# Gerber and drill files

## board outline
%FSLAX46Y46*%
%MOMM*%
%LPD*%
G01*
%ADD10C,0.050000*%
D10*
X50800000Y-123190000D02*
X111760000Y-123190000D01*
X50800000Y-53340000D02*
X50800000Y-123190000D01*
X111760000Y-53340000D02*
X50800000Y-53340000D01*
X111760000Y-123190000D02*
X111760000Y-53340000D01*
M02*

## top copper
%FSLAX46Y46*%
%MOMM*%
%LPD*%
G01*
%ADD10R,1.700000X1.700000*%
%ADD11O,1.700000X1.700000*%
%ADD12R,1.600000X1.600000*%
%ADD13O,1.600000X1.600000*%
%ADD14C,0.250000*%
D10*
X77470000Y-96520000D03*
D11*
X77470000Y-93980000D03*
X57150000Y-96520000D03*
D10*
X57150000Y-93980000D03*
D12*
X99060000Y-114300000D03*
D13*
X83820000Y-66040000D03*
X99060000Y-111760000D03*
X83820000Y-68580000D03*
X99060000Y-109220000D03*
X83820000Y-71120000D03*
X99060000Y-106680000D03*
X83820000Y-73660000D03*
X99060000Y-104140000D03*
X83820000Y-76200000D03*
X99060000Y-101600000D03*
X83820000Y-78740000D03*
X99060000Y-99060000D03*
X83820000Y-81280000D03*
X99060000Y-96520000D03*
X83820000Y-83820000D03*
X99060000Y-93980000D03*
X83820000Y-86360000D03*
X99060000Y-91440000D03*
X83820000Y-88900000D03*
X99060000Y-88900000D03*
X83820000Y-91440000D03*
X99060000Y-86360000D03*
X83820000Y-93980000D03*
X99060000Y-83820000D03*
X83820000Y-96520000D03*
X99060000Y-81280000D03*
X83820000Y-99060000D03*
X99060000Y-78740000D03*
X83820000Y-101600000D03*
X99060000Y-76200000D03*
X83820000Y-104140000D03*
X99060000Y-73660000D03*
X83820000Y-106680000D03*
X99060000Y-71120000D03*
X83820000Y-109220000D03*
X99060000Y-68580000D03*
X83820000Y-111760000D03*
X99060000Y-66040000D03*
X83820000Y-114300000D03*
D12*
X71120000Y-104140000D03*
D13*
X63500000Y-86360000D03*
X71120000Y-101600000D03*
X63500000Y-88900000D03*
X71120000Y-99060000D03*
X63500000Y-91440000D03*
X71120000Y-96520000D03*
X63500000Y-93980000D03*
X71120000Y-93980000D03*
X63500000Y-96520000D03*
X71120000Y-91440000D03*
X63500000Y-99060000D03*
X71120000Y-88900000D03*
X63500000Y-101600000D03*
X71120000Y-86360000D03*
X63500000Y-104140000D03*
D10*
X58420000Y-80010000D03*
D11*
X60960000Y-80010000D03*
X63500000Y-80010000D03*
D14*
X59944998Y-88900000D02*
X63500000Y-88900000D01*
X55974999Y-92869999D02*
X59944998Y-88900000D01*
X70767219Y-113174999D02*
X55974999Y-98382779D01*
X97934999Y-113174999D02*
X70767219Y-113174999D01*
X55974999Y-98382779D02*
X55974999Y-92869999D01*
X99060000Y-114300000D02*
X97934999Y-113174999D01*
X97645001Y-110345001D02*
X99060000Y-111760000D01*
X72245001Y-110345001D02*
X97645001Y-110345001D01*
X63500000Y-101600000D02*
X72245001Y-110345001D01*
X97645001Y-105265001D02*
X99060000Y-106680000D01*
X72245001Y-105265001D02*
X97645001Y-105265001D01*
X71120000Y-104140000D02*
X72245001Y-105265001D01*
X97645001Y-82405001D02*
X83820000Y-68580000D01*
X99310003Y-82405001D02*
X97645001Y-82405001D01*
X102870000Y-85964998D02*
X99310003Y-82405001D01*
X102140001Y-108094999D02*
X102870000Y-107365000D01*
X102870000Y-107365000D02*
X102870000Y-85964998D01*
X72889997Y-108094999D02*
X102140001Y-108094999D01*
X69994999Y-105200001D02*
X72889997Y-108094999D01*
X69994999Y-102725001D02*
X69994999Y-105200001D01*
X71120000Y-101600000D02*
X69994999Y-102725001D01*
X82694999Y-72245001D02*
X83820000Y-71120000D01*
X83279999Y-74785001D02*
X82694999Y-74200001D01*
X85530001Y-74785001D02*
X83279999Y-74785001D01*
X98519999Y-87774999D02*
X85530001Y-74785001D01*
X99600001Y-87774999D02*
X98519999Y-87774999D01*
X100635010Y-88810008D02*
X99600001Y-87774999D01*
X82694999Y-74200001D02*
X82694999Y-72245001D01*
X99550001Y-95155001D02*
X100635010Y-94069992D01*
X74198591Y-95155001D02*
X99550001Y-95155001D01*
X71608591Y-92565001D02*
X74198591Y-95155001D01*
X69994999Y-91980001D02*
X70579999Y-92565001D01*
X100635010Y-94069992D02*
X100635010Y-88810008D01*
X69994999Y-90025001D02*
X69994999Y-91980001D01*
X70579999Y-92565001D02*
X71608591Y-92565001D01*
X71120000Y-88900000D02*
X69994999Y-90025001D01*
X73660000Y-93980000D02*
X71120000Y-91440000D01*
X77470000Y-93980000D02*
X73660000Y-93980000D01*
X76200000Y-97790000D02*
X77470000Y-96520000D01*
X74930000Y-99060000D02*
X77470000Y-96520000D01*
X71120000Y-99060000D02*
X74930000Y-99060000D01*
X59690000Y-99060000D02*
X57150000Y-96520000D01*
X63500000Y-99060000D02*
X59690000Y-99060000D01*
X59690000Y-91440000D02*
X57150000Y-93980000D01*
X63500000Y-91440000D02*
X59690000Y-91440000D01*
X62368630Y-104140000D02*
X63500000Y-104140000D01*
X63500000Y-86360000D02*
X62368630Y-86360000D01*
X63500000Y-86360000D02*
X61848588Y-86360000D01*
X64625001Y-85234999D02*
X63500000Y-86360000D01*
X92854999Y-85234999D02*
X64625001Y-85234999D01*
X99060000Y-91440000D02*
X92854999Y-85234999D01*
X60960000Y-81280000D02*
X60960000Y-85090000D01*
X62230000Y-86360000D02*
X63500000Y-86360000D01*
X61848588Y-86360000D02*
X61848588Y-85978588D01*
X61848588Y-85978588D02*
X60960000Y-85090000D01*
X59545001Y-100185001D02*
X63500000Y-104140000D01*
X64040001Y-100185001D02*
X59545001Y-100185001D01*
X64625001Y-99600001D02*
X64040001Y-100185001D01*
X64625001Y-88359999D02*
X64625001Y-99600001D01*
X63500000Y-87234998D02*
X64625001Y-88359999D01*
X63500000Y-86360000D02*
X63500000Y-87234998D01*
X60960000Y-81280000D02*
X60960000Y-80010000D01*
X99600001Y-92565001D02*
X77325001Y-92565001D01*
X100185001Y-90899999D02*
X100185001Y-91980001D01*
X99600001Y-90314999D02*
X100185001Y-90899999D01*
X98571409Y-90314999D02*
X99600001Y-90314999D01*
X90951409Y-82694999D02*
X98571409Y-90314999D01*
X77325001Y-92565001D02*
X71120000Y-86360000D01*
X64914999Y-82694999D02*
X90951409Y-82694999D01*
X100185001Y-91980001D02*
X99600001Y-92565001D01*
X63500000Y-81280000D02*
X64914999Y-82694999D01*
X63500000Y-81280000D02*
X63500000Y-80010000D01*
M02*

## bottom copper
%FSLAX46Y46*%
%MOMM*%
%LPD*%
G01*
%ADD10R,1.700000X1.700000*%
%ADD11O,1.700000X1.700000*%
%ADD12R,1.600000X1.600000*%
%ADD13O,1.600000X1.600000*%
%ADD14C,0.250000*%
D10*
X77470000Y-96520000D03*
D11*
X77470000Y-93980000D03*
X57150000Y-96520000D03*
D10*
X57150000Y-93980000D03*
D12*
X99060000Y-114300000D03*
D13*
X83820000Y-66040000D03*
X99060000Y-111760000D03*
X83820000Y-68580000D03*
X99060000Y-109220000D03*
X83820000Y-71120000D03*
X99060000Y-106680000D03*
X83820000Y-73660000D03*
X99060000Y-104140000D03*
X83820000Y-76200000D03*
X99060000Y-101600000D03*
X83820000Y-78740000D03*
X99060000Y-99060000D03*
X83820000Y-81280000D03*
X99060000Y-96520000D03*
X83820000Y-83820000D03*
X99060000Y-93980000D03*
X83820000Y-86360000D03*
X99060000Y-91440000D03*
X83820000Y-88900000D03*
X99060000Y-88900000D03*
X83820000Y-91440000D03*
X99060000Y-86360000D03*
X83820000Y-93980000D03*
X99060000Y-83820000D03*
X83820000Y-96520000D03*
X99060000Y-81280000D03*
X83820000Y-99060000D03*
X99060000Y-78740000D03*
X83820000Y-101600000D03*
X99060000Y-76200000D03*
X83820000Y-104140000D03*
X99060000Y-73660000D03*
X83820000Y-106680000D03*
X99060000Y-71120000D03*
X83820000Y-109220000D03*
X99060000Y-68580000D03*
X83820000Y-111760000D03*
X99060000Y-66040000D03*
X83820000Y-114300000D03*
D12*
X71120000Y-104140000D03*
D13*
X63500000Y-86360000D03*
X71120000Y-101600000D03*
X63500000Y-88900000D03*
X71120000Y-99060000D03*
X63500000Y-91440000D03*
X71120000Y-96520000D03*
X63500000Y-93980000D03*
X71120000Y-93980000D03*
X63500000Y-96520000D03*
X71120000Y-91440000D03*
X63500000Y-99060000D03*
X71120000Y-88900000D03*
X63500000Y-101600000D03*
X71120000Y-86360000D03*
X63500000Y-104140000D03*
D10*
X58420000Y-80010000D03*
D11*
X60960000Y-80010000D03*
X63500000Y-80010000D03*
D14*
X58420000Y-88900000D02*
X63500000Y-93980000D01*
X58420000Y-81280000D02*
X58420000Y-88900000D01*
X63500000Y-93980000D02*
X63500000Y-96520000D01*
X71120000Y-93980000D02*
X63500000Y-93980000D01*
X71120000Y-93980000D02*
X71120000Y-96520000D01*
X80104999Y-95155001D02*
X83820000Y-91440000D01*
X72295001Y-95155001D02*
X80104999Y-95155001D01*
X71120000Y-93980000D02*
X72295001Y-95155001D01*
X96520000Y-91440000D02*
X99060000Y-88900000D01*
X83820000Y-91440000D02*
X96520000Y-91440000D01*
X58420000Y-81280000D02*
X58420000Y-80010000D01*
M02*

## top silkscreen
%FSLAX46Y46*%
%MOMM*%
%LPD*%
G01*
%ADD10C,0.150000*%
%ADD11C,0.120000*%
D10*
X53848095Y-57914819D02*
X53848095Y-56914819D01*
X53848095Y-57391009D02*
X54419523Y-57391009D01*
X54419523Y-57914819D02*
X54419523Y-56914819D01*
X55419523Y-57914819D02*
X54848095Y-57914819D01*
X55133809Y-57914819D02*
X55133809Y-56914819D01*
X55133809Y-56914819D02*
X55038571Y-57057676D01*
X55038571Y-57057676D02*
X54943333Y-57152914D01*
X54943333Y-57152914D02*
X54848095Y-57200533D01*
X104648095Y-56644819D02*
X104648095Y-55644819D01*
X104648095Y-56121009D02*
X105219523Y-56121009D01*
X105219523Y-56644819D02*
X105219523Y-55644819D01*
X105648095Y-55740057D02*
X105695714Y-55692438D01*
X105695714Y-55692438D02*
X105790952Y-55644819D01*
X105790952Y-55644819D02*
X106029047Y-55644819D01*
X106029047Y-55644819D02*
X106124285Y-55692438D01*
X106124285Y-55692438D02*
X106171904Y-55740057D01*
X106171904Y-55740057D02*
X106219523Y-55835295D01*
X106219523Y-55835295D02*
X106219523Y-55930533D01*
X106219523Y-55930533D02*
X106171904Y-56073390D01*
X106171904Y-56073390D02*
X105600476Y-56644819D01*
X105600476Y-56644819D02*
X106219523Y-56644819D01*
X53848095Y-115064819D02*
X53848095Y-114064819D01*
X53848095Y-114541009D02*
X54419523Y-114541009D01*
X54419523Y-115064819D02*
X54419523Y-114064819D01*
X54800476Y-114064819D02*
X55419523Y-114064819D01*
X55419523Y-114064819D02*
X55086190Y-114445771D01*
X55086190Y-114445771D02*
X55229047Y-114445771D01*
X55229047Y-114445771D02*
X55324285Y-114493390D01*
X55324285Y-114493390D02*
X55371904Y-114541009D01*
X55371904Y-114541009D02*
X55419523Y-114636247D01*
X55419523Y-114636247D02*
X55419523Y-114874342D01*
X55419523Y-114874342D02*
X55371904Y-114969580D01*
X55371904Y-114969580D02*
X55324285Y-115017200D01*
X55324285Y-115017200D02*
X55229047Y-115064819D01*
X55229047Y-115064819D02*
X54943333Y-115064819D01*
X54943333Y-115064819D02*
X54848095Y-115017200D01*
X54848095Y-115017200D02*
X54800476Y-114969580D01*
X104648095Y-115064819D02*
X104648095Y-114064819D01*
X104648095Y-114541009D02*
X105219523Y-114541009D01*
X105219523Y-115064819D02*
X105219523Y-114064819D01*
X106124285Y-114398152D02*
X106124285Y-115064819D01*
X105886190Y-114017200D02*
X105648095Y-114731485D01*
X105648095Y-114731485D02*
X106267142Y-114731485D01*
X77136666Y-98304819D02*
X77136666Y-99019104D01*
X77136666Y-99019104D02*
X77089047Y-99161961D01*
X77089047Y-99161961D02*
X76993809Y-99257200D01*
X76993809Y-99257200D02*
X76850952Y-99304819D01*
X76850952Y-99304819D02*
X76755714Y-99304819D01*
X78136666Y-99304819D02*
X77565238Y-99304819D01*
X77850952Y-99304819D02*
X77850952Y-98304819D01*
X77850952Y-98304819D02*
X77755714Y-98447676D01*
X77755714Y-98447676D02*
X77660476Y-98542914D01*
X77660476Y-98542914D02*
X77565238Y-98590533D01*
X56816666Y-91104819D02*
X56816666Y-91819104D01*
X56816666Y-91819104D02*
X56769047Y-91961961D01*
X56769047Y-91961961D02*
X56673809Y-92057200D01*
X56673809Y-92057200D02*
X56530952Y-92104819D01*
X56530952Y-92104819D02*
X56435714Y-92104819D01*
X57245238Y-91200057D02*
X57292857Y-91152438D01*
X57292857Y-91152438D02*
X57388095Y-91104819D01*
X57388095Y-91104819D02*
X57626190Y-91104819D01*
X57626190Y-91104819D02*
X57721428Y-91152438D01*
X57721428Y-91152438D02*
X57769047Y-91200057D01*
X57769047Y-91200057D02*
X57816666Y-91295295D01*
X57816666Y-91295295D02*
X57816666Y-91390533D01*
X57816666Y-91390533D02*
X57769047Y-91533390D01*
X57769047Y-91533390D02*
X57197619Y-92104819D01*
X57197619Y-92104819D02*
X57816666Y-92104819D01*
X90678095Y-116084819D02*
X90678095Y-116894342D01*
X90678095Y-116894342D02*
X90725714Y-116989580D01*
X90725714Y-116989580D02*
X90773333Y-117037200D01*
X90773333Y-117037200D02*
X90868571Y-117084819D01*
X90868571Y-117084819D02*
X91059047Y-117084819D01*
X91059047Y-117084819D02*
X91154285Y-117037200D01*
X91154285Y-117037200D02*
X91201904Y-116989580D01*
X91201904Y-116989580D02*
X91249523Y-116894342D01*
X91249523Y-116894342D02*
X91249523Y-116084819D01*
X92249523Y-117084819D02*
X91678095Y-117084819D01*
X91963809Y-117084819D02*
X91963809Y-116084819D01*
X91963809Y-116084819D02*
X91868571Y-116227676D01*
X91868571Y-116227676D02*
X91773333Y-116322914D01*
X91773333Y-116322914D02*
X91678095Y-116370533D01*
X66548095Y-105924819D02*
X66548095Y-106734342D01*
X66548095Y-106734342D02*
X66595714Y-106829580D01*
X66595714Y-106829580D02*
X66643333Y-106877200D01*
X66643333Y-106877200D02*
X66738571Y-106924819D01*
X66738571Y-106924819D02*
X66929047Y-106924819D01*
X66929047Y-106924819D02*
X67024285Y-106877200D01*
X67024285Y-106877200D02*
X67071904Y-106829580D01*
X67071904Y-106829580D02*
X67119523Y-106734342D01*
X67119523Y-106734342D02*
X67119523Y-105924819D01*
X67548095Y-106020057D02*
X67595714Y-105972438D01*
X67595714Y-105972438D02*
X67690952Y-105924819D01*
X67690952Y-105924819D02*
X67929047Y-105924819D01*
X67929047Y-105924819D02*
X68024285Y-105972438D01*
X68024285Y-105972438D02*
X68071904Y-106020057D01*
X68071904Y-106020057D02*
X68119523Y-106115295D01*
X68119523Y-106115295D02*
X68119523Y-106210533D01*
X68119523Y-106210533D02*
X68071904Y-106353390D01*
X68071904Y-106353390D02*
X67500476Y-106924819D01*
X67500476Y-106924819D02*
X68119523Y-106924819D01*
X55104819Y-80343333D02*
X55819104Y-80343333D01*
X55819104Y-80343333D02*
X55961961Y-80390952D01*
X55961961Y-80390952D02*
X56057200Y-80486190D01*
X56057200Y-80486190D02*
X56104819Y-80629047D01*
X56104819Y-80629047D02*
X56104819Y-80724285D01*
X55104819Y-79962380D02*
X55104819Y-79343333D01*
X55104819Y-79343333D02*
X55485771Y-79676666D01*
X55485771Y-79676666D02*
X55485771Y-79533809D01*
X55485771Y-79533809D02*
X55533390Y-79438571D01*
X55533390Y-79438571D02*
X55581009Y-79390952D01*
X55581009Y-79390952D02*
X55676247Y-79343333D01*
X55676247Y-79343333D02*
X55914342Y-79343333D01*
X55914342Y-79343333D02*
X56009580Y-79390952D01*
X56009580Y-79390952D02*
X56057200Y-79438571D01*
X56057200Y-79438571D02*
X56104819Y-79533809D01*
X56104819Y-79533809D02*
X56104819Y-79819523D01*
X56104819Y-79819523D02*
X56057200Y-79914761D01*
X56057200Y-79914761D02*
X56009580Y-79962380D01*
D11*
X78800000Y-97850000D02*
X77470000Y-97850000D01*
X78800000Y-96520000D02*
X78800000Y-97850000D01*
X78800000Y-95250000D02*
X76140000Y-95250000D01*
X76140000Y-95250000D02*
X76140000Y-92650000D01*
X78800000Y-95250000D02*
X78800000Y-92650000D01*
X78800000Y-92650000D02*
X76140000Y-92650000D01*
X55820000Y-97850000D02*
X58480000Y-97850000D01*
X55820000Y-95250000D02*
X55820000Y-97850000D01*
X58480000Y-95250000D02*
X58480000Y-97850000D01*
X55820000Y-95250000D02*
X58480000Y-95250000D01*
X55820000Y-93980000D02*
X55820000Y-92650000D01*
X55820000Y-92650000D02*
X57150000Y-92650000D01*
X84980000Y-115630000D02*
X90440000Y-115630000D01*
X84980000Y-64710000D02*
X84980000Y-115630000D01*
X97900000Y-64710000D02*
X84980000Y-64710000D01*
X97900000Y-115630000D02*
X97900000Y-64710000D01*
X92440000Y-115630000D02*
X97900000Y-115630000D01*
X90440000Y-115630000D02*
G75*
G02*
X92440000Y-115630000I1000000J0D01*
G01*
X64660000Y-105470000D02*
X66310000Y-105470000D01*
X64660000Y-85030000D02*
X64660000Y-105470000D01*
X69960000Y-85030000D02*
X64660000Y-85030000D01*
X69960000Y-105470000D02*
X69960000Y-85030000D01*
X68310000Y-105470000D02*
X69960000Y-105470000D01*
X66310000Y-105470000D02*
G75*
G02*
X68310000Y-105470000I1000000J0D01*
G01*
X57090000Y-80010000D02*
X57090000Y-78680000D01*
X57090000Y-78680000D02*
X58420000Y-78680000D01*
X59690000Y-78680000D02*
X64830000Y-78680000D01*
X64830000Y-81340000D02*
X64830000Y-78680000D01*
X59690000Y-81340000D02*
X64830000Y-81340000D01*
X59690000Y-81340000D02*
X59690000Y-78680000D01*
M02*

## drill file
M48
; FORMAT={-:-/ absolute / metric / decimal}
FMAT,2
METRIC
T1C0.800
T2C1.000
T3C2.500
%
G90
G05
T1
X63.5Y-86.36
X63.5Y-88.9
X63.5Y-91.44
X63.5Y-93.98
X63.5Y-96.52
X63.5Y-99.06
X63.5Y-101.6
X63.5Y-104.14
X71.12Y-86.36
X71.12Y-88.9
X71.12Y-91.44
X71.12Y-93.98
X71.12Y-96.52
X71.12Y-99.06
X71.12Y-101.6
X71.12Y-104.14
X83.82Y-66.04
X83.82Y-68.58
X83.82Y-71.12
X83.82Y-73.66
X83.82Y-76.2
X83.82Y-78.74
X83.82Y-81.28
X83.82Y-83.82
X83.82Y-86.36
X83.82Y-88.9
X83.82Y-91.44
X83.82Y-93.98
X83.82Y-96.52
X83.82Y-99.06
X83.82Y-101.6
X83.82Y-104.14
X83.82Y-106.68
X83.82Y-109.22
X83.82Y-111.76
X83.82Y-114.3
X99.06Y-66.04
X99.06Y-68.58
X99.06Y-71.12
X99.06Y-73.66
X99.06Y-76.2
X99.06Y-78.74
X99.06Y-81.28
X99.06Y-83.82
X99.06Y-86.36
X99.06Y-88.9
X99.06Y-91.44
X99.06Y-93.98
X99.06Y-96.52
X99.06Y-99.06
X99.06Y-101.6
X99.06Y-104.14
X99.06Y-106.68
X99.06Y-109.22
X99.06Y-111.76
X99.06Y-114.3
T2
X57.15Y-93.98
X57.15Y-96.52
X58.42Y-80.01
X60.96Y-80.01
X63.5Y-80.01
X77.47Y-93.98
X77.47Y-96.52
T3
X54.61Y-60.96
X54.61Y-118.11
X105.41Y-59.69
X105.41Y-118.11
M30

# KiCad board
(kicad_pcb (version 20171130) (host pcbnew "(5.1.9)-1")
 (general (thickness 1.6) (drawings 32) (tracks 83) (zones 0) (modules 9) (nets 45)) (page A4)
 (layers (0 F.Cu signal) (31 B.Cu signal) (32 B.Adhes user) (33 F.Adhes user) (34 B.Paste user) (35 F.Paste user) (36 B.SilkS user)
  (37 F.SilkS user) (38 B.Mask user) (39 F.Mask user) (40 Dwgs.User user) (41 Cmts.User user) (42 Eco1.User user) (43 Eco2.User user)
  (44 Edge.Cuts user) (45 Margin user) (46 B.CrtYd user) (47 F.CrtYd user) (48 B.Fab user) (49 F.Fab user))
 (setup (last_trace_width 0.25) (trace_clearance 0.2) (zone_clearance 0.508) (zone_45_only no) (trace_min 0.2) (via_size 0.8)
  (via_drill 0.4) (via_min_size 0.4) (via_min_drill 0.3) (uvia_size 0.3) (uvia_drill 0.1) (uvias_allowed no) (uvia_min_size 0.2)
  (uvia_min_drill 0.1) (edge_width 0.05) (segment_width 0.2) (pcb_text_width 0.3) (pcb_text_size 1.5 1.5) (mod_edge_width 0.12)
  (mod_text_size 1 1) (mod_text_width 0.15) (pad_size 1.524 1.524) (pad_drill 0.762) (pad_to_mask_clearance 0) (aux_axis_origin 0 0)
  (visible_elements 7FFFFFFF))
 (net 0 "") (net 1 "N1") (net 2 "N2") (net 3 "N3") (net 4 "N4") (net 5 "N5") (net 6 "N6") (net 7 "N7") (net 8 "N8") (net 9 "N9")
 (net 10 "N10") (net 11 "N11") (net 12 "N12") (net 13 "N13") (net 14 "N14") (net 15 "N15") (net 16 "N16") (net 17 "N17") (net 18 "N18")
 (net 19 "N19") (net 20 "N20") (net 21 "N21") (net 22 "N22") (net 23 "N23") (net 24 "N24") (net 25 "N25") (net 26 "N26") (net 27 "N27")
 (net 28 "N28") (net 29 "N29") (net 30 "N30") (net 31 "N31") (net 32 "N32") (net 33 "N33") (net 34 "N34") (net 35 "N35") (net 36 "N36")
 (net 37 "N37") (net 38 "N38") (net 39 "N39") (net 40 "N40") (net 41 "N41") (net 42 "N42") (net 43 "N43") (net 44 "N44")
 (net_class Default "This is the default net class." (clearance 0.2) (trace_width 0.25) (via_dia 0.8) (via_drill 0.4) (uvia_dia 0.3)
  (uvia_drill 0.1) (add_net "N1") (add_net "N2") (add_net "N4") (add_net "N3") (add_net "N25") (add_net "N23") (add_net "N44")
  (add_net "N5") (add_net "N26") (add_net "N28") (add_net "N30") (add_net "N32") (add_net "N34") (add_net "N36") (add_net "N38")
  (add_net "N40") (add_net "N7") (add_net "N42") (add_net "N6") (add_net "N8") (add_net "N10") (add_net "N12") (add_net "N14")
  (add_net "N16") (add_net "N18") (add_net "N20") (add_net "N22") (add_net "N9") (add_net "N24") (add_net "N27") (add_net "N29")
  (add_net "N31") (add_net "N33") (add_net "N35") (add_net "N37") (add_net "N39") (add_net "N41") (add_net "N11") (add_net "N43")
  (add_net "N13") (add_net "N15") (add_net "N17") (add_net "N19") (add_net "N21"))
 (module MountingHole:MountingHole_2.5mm (layer F.Cu) (at 54.61 60.96)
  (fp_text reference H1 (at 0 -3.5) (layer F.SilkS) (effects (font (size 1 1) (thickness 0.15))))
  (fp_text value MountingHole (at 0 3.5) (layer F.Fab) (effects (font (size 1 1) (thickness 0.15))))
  (pad 1 np_thru_hole circle (at 0 0) (size 2.5 2.5) (drill 2.5) (layers *.Cu *.Mask)))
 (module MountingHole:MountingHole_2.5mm (layer F.Cu) (at 105.41 59.69)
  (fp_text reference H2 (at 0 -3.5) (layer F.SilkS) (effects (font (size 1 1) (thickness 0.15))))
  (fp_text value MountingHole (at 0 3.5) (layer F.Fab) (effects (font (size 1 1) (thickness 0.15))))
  (pad 1 np_thru_hole circle (at 0 0) (size 2.5 2.5) (drill 2.5) (layers *.Cu *.Mask)))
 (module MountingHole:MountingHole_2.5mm (layer F.Cu) (at 54.61 118.11)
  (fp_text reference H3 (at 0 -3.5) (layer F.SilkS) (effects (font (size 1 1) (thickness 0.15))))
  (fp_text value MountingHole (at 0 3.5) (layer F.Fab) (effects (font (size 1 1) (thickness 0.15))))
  (pad 1 np_thru_hole circle (at 0 0) (size 2.5 2.5) (drill 2.5) (layers *.Cu *.Mask)))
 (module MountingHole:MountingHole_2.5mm (layer F.Cu) (at 105.41 118.11)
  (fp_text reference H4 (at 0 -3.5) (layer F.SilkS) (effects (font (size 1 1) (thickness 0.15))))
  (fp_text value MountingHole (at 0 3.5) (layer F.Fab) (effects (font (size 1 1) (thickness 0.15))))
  (pad 1 np_thru_hole circle (at 0 0) (size 2.5 2.5) (drill 2.5) (layers *.Cu *.Mask)))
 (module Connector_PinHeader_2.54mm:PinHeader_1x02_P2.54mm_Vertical (layer F.Cu) (at 77.47 96.52 180)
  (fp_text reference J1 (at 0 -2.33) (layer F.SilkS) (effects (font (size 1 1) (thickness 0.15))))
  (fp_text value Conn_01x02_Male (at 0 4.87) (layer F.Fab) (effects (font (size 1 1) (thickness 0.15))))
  (fp_line (start -1.33 -1.33) (end 0 -1.33) (layer F.SilkS) (width 0.12))
  (fp_line (start -1.33 0) (end -1.33 -1.33) (layer F.SilkS) (width 0.12))
  (fp_line (start -1.33 1.27) (end 1.33 1.27) (layer F.SilkS) (width 0.12))
  (fp_line (start 1.33 1.27) (end 1.33 3.87) (layer F.SilkS) (width 0.12))
  (fp_line (start -1.33 1.27) (end -1.33 3.87) (layer F.SilkS) (width 0.12))
  (fp_line (start -1.33 3.87) (end 1.33 3.87) (layer F.SilkS) (width 0.12))
  (pad 1 thru_hole rect (at 0 0 180) (size 1.7 1.7) (drill 1) (layers *.Cu *.Mask) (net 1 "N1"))
  (pad 2 thru_hole oval (at 0 2.54 180) (size 1.7 1.7) (drill 1) (layers *.Cu *.Mask) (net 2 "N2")))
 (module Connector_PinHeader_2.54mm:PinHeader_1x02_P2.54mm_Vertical (layer F.Cu) (at 57.15 93.98)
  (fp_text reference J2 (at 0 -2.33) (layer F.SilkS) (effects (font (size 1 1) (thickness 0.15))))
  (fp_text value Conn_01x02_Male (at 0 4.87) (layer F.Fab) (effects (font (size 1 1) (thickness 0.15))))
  (fp_line (start -1.33 3.87) (end 1.33 3.87) (layer F.SilkS) (width 0.12))
  (fp_line (start -1.33 1.27) (end -1.33 3.87) (layer F.SilkS) (width 0.12))
  (fp_line (start 1.33 1.27) (end 1.33 3.87) (layer F.SilkS) (width 0.12))
  (fp_line (start -1.33 1.27) (end 1.33 1.27) (layer F.SilkS) (width 0.12))
  (fp_line (start -1.33 0) (end -1.33 -1.33) (layer F.SilkS) (width 0.12))
  (fp_line (start -1.33 -1.33) (end 0 -1.33) (layer F.SilkS) (width 0.12))
  (pad 2 thru_hole oval (at 0 2.54) (size 1.7 1.7) (drill 1) (layers *.Cu *.Mask) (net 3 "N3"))
  (pad 1 thru_hole rect (at 0 0) (size 1.7 1.7) (drill 1) (layers *.Cu *.Mask) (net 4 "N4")))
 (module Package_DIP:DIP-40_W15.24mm (layer F.Cu) (at 99.06 114.3 180)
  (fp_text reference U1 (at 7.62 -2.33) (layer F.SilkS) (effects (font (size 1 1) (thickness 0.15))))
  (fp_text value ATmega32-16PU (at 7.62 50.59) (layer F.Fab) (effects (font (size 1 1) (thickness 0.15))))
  (fp_line (start 14.08 -1.33) (end 8.62 -1.33) (layer F.SilkS) (width 0.12))
  (fp_line (start 14.08 49.59) (end 14.08 -1.33) (layer F.SilkS) (width 0.12))
  (fp_line (start 1.16 49.59) (end 14.08 49.59) (layer F.SilkS) (width 0.12))
  (fp_line (start 1.16 -1.33) (end 1.16 49.59) (layer F.SilkS) (width 0.12))
  (fp_line (start 6.62 -1.33) (end 1.16 -1.33) (layer F.SilkS) (width 0.12))
  (fp_arc (start 7.62 -1.33) (end 6.62 -1.33) (angle -180) (layer F.SilkS) (width 0.12))
  (pad 1 thru_hole rect (at 0 0 180) (size 1.6 1.6) (drill 0.8) (layers *.Cu *.Mask) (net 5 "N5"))
  (pad 21 thru_hole oval (at 15.24 48.26 180) (size 1.6 1.6) (drill 0.8) (layers *.Cu *.Mask) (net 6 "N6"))
  (pad 2 thru_hole oval (at 0 2.54 180) (size 1.6 1.6) (drill 0.8) (layers *.Cu *.Mask) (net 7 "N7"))
  (pad 22 thru_hole oval (at 15.24 45.72 180) (size 1.6 1.6) (drill 0.8) (layers *.Cu *.Mask) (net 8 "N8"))
  (pad 3 thru_hole oval (at 0 5.08 180) (size 1.6 1.6) (drill 0.8) (layers *.Cu *.Mask) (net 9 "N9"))
  (pad 23 thru_hole oval (at 15.24 43.18 180) (size 1.6 1.6) (drill 0.8) (layers *.Cu *.Mask) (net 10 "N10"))
  (pad 4 thru_hole oval (at 0 7.62 180) (size 1.6 1.6) (drill 0.8) (layers *.Cu *.Mask) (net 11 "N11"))
  (pad 24 thru_hole oval (at 15.24 40.64 180) (size 1.6 1.6) (drill 0.8) (layers *.Cu *.Mask) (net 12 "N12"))
  (pad 5 thru_hole oval (at 0 10.16 180) (size 1.6 1.6) (drill 0.8) (layers *.Cu *.Mask) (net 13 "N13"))
  (pad 25 thru_hole oval (at 15.24 38.1 180) (size 1.6 1.6) (drill 0.8) (layers *.Cu *.Mask) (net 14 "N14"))
  (pad 6 thru_hole oval (at 0 12.7 180) (size 1.6 1.6) (drill 0.8) (layers *.Cu *.Mask) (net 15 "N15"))
  (pad 26 thru_hole oval (at 15.24 35.56 180) (size 1.6 1.6) (drill 0.8) (layers *.Cu *.Mask) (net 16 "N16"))
  (pad 7 thru_hole oval (at 0 15.24 180) (size 1.6 1.6) (drill 0.8) (layers *.Cu *.Mask) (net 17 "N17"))
  (pad 27 thru_hole oval (at 15.24 33.02 180) (size 1.6 1.6) (drill 0.8) (layers *.Cu *.Mask) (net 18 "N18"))
  (pad 8 thru_hole oval (at 0 17.78 180) (size 1.6 1.6) (drill 0.8) (layers *.Cu *.Mask) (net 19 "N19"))
  (pad 28 thru_hole oval (at 15.24 30.48 180) (size 1.6 1.6) (drill 0.8) (layers *.Cu *.Mask) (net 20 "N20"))
  (pad 9 thru_hole oval (at 0 20.32 180) (size 1.6 1.6) (drill 0.8) (layers *.Cu *.Mask) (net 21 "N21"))
  (pad 29 thru_hole oval (at 15.24 27.94 180) (size 1.6 1.6) (drill 0.8) (layers *.Cu *.Mask) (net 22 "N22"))
  (pad 10 thru_hole oval (at 0 22.86 180) (size 1.6 1.6) (drill 0.8) (layers *.Cu *.Mask) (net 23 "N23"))
  (pad 30 thru_hole oval (at 15.24 25.4 180) (size 1.6 1.6) (drill 0.8) (layers *.Cu *.Mask) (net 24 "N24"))
  (pad 11 thru_hole oval (at 0 25.4 180) (size 1.6 1.6) (drill 0.8) (layers *.Cu *.Mask) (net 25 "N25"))
  (pad 31 thru_hole oval (at 15.24 22.86 180) (size 1.6 1.6) (drill 0.8) (layers *.Cu *.Mask) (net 25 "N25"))
  (pad 12 thru_hole oval (at 0 27.94 180) (size 1.6 1.6) (drill 0.8) (layers *.Cu *.Mask) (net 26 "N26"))
  (pad 32 thru_hole oval (at 15.24 20.32 180) (size 1.6 1.6) (drill 0.8) (layers *.Cu *.Mask) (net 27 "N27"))
  (pad 13 thru_hole oval (at 0 30.48 180) (size 1.6 1.6) (drill 0.8) (layers *.Cu *.Mask) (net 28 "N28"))
  (pad 33 thru_hole oval (at 15.24 17.78 180) (size 1.6 1.6) (drill 0.8) (layers *.Cu *.Mask) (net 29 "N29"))
  (pad 14 thru_hole oval (at 0 33.02 180) (size 1.6 1.6) (drill 0.8) (layers *.Cu *.Mask) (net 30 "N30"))
  (pad 34 thru_hole oval (at 15.24 15.24 180) (size 1.6 1.6) (drill 0.8) (layers *.Cu *.Mask) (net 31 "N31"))
  (pad 15 thru_hole oval (at 0 35.56 180) (size 1.6 1.6) (drill 0.8) (layers *.Cu *.Mask) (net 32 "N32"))
  (pad 35 thru_hole oval (at 15.24 12.7 180) (size 1.6 1.6) (drill 0.8) (layers *.Cu *.Mask) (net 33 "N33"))
  (pad 16 thru_hole oval (at 0 38.1 180) (size 1.6 1.6) (drill 0.8) (layers *.Cu *.Mask) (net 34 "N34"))
  (pad 36 thru_hole oval (at 15.24 10.16 180) (size 1.6 1.6) (drill 0.8) (layers *.Cu *.Mask) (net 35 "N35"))
  (pad 17 thru_hole oval (at 0 40.64 180) (size 1.6 1.6) (drill 0.8) (layers *.Cu *.Mask) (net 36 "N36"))
  (pad 37 thru_hole oval (at 15.24 7.62 180) (size 1.6 1.6) (drill 0.8) (layers *.Cu *.Mask) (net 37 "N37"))
  (pad 18 thru_hole oval (at 0 43.18 180) (size 1.6 1.6) (drill 0.8) (layers *.Cu *.Mask) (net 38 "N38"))
  (pad 38 thru_hole oval (at 15.24 5.08 180) (size 1.6 1.6) (drill 0.8) (layers *.Cu *.Mask) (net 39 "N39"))
  (pad 19 thru_hole oval (at 0 45.72 180) (size 1.6 1.6) (drill 0.8) (layers *.Cu *.Mask) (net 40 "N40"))
  (pad 39 thru_hole oval (at 15.24 2.54 180) (size 1.6 1.6) (drill 0.8) (layers *.Cu *.Mask) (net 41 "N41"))
  (pad 20 thru_hole oval (at 0 48.26 180) (size 1.6 1.6) (drill 0.8) (layers *.Cu *.Mask) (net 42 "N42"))
  (pad 40 thru_hole oval (at 15.24 0 180) (size 1.6 1.6) (drill 0.8) (layers *.Cu *.Mask) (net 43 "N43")))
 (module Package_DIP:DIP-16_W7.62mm (layer F.Cu) (at 71.12 104.14 180)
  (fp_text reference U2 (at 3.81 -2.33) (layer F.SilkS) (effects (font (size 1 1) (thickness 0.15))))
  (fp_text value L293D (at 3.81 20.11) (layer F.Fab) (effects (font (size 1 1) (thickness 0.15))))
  (fp_line (start 6.46 -1.33) (end 4.81 -1.33) (layer F.SilkS) (width 0.12))
  (fp_line (start 6.46 19.11) (end 6.46 -1.33) (layer F.SilkS) (width 0.12))
  (fp_line (start 1.16 19.11) (end 6.46 19.11) (layer F.SilkS) (width 0.12))
  (fp_line (start 1.16 -1.33) (end 1.16 19.11) (layer F.SilkS) (width 0.12))
  (fp_line (start 2.81 -1.33) (end 1.16 -1.33) (layer F.SilkS) (width 0.12))
  (fp_arc (start 3.81 -1.33) (end 2.81 -1.33) (angle -180) (layer F.SilkS) (width 0.12))
  (pad 1 thru_hole rect (at 0 0 180) (size 1.6 1.6) (drill 0.8) (layers *.Cu *.Mask) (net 11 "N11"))
  (pad 9 thru_hole oval (at 7.62 17.78 180) (size 1.6 1.6) (drill 0.8) (layers *.Cu *.Mask) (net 23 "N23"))
  (pad 2 thru_hole oval (at 0 2.54 180) (size 1.6 1.6) (drill 0.8) (layers *.Cu *.Mask) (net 8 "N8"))
  (pad 10 thru_hole oval (at 7.62 15.24 180) (size 1.6 1.6) (drill 0.8) (layers *.Cu *.Mask) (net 5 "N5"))
  (pad 3 thru_hole oval (at 0 5.08 180) (size 1.6 1.6) (drill 0.8) (layers *.Cu *.Mask) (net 1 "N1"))
  (pad 11 thru_hole oval (at 7.62 12.7 180) (size 1.6 1.6) (drill 0.8) (layers *.Cu *.Mask) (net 4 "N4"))
  (pad 4 thru_hole oval (at 0 7.62 180) (size 1.6 1.6) (drill 0.8) (layers *.Cu *.Mask) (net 25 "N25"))
  (pad 12 thru_hole oval (at 7.62 10.16 180) (size 1.6 1.6) (drill 0.8) (layers *.Cu *.Mask) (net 25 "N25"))
  (pad 5 thru_hole oval (at 0 10.16 180) (size 1.6 1.6) (drill 0.8) (layers *.Cu *.Mask) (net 25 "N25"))
  (pad 13 thru_hole oval (at 7.62 7.62 180) (size 1.6 1.6) (drill 0.8) (layers *.Cu *.Mask) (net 25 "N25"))
  (pad 6 thru_hole oval (at 0 12.7 180) (size 1.6 1.6) (drill 0.8) (layers *.Cu *.Mask) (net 2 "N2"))
  (pad 14 thru_hole oval (at 7.62 5.08 180) (size 1.6 1.6) (drill 0.8) (layers *.Cu *.Mask) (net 3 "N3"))
  (pad 7 thru_hole oval (at 0 15.24 180) (size 1.6 1.6) (drill 0.8) (layers *.Cu *.Mask) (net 10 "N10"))
  (pad 15 thru_hole oval (at 7.62 2.54 180) (size 1.6 1.6) (drill 0.8) (layers *.Cu *.Mask) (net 7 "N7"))
  (pad 8 thru_hole oval (at 0 17.78 180) (size 1.6 1.6) (drill 0.8) (layers *.Cu *.Mask) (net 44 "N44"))
  (pad 16 thru_hole oval (at 7.62 0 180) (size 1.6 1.6) (drill 0.8) (layers *.Cu *.Mask) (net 23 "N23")))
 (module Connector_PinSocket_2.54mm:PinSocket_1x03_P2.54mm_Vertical (layer F.Cu) (at 58.42 80.01 90)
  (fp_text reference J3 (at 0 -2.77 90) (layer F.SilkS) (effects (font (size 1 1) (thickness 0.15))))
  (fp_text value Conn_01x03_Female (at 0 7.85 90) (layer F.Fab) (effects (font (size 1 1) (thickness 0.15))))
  (fp_line (start 0 -1.33) (end 1.33 -1.33) (layer F.SilkS) (width 0.12))
  (fp_line (start 1.33 -1.33) (end 1.33 0) (layer F.SilkS) (width 0.12))
  (fp_line (start 1.33 1.27) (end 1.33 6.41) (layer F.SilkS) (width 0.12))
  (fp_line (start -1.33 6.41) (end 1.33 6.41) (layer F.SilkS) (width 0.12))
  (fp_line (start -1.33 1.27) (end -1.33 6.41) (layer F.SilkS) (width 0.12))
  (fp_line (start -1.33 1.27) (end 1.33 1.27) (layer F.SilkS) (width 0.12))
  (pad 1 thru_hole rect (at 0 0 90) (size 1.7 1.7) (drill 1) (layers *.Cu *.Mask) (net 25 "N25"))
  (pad 2 thru_hole oval (at 0 2.54 90) (size 1.7 1.7) (drill 1) (layers *.Cu *.Mask) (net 23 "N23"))
  (pad 3 thru_hole oval (at 0 5.08 90) (size 1.7 1.7) (drill 1) (layers *.Cu *.Mask) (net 44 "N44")))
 (gr_line (start 50.8 123.19) (end 111.76 123.19) (layer Edge.Cuts) (width 0.05))
 (gr_line (start 50.8 53.34) (end 50.8 123.19) (layer Edge.Cuts) (width 0.05))
 (gr_line (start 111.76 53.34) (end 50.8 53.34) (layer Edge.Cuts) (width 0.05))
 (gr_line (start 111.76 123.19) (end 111.76 53.34) (layer Edge.Cuts) (width 0.05))
 (segment (start 59.944998 88.9) (end 63.5 88.9) (width 0.25) (layer F.Cu) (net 5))
 (segment (start 55.974999 92.869999) (end 59.944998 88.9) (width 0.25) (layer F.Cu) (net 5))
 (segment (start 70.767219 113.174999) (end 55.974999 98.382779) (width 0.25) (layer F.Cu) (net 5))
 (segment (start 97.934999 113.174999) (end 70.767219 113.174999) (width 0.25) (layer F.Cu) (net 5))
 (segment (start 55.974999 98.382779) (end 55.974999 92.869999) (width 0.25) (layer F.Cu) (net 5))
 (segment (start 99.06 114.3) (end 97.934999 113.174999) (width 0.25) (layer F.Cu) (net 5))
 (segment (start 97.645001 110.345001) (end 99.06 111.76) (width 0.25) (layer F.Cu) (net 7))
 (segment (start 72.245001 110.345001) (end 97.645001 110.345001) (width 0.25) (layer F.Cu) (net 7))
 (segment (start 63.5 101.6) (end 72.245001 110.345001) (width 0.25) (layer F.Cu) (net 7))
 (segment (start 97.645001 105.265001) (end 99.06 106.68) (width 0.25) (layer F.Cu) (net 11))
 (segment (start 72.245001 105.265001) (end 97.645001 105.265001) (width 0.25) (layer F.Cu) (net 11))
 (segment (start 71.12 104.14) (end 72.245001 105.265001) (width 0.25) (layer F.Cu) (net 11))
 (segment (start 97.645001 82.405001) (end 83.82 68.58) (width 0.25) (layer F.Cu) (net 8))
 (segment (start 99.310003 82.405001) (end 97.645001 82.405001) (width 0.25) (layer F.Cu) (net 8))
 (segment (start 102.87 85.964998) (end 99.310003 82.405001) (width 0.25) (layer F.Cu) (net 8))
 (segment (start 102.140001 108.094999) (end 102.87 107.365) (width 0.25) (layer F.Cu) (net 8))
 (segment (start 102.87 107.365) (end 102.87 85.964998) (width 0.25) (layer F.Cu) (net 8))
 (segment (start 72.889997 108.094999) (end 102.140001 108.094999) (width 0.25) (layer F.Cu) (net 8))
 (segment (start 69.994999 105.200001) (end 72.889997 108.094999) (width 0.25) (layer F.Cu) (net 8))
 (segment (start 69.994999 102.725001) (end 69.994999 105.200001) (width 0.25) (layer F.Cu) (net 8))
 (segment (start 71.12 101.6) (end 69.994999 102.725001) (width 0.25) (layer F.Cu) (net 8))
 (segment (start 82.694999 72.245001) (end 83.82 71.12) (width 0.25) (layer F.Cu) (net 10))
 (segment (start 83.279999 74.785001) (end 82.694999 74.200001) (width 0.25) (layer F.Cu) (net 10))
 (segment (start 85.530001 74.785001) (end 83.279999 74.785001) (width 0.25) (layer F.Cu) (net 10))
 (segment (start 98.519999 87.774999) (end 85.530001 74.785001) (width 0.25) (layer F.Cu) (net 10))
 (segment (start 99.600001 87.774999) (end 98.519999 87.774999) (width 0.25) (layer F.Cu) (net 10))
 (segment (start 100.63501 88.810008) (end 99.600001 87.774999) (width 0.25) (layer F.Cu) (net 10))
 (segment (start 82.694999 74.200001) (end 82.694999 72.245001) (width 0.25) (layer F.Cu) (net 10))
 (segment (start 99.550001 95.155001) (end 100.63501 94.069992) (width 0.25) (layer F.Cu) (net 10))
 (segment (start 74.198591 95.155001) (end 99.550001 95.155001) (width 0.25) (layer F.Cu) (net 10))
 (segment (start 71.608591 92.565001) (end 74.198591 95.155001) (width 0.25) (layer F.Cu) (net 10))
 (segment (start 69.994999 91.980001) (end 70.579999 92.565001) (width 0.25) (layer F.Cu) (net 10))
 (segment (start 100.63501 94.069992) (end 100.63501 88.810008) (width 0.25) (layer F.Cu) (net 10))
 (segment (start 69.994999 90.025001) (end 69.994999 91.980001) (width 0.25) (layer F.Cu) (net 10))
 (segment (start 70.579999 92.565001) (end 71.608591 92.565001) (width 0.25) (layer F.Cu) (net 10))
 (segment (start 71.12 88.9) (end 69.994999 90.025001) (width 0.25) (layer F.Cu) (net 10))
 (segment (start 73.66 93.98) (end 71.12 91.44) (width 0.25) (layer F.Cu) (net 2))
 (segment (start 77.47 93.98) (end 73.66 93.98) (width 0.25) (layer F.Cu) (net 2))
 (segment (start 76.2 97.79) (end 77.47 96.52) (width 0.25) (layer F.Cu) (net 1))
 (segment (start 74.93 99.06) (end 77.47 96.52) (width 0.25) (layer F.Cu) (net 1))
 (segment (start 71.12 99.06) (end 74.93 99.06) (width 0.25) (layer F.Cu) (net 1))
 (segment (start 59.69 99.06) (end 57.15 96.52) (width 0.25) (layer F.Cu) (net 3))
 (segment (start 63.5 99.06) (end 59.69 99.06) (width 0.25) (layer F.Cu) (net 3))
 (segment (start 59.69 91.44) (end 57.15 93.98) (width 0.25) (layer F.Cu) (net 4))
 (segment (start 63.5 91.44) (end 59.69 91.44) (width 0.25) (layer F.Cu) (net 4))
 (segment (start 58.42 88.9) (end 63.5 93.98) (width 0.25) (layer B.Cu) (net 25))
 (segment (start 58.42 81.28) (end 58.42 88.9) (width 0.25) (layer B.Cu) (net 25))
 (segment (start 63.5 93.98) (end 63.5 96.52) (width 0.25) (layer B.Cu) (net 25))
 (segment (start 71.12 93.98) (end 63.5 93.98) (width 0.25) (layer B.Cu) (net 25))
 (segment (start 71.12 93.98) (end 71.12 96.52) (width 0.25) (layer B.Cu) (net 25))
 (segment (start 80.104999 95.155001) (end 83.82 91.44) (width 0.25) (layer B.Cu) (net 25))
 (segment (start 72.295001 95.155001) (end 80.104999 95.155001) (width 0.25) (layer B.Cu) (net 25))
 (segment (start 71.12 93.98) (end 72.295001 95.155001) (width 0.25) (layer B.Cu) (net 25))
 (segment (start 96.52 91.44) (end 99.06 88.9) (width 0.25) (layer B.Cu) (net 25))
 (segment (start 83.82 91.44) (end 96.52 91.44) (width 0.25) (layer B.Cu) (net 25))
 (segment (start 58.42 81.28) (end 58.42 80.01) (width 0.25) (layer B.Cu) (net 25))
 (segment (start 62.36863 104.14) (end 63.5 104.14) (width 0.25) (layer F.Cu) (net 23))
 (segment (start 63.5 86.36) (end 62.36863 86.36) (width 0.25) (layer F.Cu) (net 23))
 (segment (start 63.5 86.36) (end 61.848588 86.36) (width 0.25) (layer F.Cu) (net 23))
 (segment (start 64.625001 85.234999) (end 63.5 86.36) (width 0.25) (layer F.Cu) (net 23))
 (segment (start 92.854999 85.234999) (end 64.625001 85.234999) (width 0.25) (layer F.Cu) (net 23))
 (segment (start 99.06 91.44) (end 92.854999 85.234999) (width 0.25) (layer F.Cu) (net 23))
 (segment (start 60.96 81.28) (end 60.96 85.09) (width 0.25) (layer F.Cu) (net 23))
 (segment (start 62.23 86.36) (end 63.5 86.36) (width 0.25) (layer F.Cu) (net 23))
 (segment (start 61.848588 86.36) (end 61.848588 85.978588) (width 0.25) (layer F.Cu) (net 23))
 (segment (start 61.848588 85.978588) (end 60.96 85.09) (width 0.25) (layer F.Cu) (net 23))
 (segment (start 59.545001 100.185001) (end 63.5 104.14) (width 0.25) (layer F.Cu) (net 23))
 (segment (start 64.040001 100.185001) (end 59.545001 100.185001) (width 0.25) (layer F.Cu) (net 23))
 (segment (start 64.625001 99.600001) (end 64.040001 100.185001) (width 0.25) (layer F.Cu) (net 23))
 (segment (start 64.625001 88.359999) (end 64.625001 99.600001) (width 0.25) (layer F.Cu) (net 23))
 (segment (start 63.5 87.234998) (end 64.625001 88.359999) (width 0.25) (layer F.Cu) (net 23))
 (segment (start 63.5 86.36) (end 63.5 87.234998) (width 0.25) (layer F.Cu) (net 23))
 (segment (start 60.96 81.28) (end 60.96 80.01) (width 0.25) (layer F.Cu) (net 23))
 (segment (start 99.600001 92.565001) (end 77.325001 92.565001) (width 0.25) (layer F.Cu) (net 44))
 (segment (start 100.185001 90.899999) (end 100.185001 91.980001) (width 0.25) (layer F.Cu) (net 44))
 (segment (start 99.600001 90.314999) (end 100.185001 90.899999) (width 0.25) (layer F.Cu) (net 44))
 (segment (start 98.571409 90.314999) (end 99.600001 90.314999) (width 0.25) (layer F.Cu) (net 44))
 (segment (start 90.951409 82.694999) (end 98.571409 90.314999) (width 0.25) (layer F.Cu) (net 44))
 (segment (start 77.325001 92.565001) (end 71.12 86.36) (width 0.25) (layer F.Cu) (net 44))
 (segment (start 64.914999 82.694999) (end 90.951409 82.694999) (width 0.25) (layer F.Cu) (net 44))
 (segment (start 100.185001 91.980001) (end 99.600001 92.565001) (width 0.25) (layer F.Cu) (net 44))
 (segment (start 63.5 81.28) (end 64.914999 82.694999) (width 0.25) (layer F.Cu) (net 44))
 (segment (start 63.5 81.28) (end 63.5 80.01) (width 0.25) (layer F.Cu) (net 44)))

